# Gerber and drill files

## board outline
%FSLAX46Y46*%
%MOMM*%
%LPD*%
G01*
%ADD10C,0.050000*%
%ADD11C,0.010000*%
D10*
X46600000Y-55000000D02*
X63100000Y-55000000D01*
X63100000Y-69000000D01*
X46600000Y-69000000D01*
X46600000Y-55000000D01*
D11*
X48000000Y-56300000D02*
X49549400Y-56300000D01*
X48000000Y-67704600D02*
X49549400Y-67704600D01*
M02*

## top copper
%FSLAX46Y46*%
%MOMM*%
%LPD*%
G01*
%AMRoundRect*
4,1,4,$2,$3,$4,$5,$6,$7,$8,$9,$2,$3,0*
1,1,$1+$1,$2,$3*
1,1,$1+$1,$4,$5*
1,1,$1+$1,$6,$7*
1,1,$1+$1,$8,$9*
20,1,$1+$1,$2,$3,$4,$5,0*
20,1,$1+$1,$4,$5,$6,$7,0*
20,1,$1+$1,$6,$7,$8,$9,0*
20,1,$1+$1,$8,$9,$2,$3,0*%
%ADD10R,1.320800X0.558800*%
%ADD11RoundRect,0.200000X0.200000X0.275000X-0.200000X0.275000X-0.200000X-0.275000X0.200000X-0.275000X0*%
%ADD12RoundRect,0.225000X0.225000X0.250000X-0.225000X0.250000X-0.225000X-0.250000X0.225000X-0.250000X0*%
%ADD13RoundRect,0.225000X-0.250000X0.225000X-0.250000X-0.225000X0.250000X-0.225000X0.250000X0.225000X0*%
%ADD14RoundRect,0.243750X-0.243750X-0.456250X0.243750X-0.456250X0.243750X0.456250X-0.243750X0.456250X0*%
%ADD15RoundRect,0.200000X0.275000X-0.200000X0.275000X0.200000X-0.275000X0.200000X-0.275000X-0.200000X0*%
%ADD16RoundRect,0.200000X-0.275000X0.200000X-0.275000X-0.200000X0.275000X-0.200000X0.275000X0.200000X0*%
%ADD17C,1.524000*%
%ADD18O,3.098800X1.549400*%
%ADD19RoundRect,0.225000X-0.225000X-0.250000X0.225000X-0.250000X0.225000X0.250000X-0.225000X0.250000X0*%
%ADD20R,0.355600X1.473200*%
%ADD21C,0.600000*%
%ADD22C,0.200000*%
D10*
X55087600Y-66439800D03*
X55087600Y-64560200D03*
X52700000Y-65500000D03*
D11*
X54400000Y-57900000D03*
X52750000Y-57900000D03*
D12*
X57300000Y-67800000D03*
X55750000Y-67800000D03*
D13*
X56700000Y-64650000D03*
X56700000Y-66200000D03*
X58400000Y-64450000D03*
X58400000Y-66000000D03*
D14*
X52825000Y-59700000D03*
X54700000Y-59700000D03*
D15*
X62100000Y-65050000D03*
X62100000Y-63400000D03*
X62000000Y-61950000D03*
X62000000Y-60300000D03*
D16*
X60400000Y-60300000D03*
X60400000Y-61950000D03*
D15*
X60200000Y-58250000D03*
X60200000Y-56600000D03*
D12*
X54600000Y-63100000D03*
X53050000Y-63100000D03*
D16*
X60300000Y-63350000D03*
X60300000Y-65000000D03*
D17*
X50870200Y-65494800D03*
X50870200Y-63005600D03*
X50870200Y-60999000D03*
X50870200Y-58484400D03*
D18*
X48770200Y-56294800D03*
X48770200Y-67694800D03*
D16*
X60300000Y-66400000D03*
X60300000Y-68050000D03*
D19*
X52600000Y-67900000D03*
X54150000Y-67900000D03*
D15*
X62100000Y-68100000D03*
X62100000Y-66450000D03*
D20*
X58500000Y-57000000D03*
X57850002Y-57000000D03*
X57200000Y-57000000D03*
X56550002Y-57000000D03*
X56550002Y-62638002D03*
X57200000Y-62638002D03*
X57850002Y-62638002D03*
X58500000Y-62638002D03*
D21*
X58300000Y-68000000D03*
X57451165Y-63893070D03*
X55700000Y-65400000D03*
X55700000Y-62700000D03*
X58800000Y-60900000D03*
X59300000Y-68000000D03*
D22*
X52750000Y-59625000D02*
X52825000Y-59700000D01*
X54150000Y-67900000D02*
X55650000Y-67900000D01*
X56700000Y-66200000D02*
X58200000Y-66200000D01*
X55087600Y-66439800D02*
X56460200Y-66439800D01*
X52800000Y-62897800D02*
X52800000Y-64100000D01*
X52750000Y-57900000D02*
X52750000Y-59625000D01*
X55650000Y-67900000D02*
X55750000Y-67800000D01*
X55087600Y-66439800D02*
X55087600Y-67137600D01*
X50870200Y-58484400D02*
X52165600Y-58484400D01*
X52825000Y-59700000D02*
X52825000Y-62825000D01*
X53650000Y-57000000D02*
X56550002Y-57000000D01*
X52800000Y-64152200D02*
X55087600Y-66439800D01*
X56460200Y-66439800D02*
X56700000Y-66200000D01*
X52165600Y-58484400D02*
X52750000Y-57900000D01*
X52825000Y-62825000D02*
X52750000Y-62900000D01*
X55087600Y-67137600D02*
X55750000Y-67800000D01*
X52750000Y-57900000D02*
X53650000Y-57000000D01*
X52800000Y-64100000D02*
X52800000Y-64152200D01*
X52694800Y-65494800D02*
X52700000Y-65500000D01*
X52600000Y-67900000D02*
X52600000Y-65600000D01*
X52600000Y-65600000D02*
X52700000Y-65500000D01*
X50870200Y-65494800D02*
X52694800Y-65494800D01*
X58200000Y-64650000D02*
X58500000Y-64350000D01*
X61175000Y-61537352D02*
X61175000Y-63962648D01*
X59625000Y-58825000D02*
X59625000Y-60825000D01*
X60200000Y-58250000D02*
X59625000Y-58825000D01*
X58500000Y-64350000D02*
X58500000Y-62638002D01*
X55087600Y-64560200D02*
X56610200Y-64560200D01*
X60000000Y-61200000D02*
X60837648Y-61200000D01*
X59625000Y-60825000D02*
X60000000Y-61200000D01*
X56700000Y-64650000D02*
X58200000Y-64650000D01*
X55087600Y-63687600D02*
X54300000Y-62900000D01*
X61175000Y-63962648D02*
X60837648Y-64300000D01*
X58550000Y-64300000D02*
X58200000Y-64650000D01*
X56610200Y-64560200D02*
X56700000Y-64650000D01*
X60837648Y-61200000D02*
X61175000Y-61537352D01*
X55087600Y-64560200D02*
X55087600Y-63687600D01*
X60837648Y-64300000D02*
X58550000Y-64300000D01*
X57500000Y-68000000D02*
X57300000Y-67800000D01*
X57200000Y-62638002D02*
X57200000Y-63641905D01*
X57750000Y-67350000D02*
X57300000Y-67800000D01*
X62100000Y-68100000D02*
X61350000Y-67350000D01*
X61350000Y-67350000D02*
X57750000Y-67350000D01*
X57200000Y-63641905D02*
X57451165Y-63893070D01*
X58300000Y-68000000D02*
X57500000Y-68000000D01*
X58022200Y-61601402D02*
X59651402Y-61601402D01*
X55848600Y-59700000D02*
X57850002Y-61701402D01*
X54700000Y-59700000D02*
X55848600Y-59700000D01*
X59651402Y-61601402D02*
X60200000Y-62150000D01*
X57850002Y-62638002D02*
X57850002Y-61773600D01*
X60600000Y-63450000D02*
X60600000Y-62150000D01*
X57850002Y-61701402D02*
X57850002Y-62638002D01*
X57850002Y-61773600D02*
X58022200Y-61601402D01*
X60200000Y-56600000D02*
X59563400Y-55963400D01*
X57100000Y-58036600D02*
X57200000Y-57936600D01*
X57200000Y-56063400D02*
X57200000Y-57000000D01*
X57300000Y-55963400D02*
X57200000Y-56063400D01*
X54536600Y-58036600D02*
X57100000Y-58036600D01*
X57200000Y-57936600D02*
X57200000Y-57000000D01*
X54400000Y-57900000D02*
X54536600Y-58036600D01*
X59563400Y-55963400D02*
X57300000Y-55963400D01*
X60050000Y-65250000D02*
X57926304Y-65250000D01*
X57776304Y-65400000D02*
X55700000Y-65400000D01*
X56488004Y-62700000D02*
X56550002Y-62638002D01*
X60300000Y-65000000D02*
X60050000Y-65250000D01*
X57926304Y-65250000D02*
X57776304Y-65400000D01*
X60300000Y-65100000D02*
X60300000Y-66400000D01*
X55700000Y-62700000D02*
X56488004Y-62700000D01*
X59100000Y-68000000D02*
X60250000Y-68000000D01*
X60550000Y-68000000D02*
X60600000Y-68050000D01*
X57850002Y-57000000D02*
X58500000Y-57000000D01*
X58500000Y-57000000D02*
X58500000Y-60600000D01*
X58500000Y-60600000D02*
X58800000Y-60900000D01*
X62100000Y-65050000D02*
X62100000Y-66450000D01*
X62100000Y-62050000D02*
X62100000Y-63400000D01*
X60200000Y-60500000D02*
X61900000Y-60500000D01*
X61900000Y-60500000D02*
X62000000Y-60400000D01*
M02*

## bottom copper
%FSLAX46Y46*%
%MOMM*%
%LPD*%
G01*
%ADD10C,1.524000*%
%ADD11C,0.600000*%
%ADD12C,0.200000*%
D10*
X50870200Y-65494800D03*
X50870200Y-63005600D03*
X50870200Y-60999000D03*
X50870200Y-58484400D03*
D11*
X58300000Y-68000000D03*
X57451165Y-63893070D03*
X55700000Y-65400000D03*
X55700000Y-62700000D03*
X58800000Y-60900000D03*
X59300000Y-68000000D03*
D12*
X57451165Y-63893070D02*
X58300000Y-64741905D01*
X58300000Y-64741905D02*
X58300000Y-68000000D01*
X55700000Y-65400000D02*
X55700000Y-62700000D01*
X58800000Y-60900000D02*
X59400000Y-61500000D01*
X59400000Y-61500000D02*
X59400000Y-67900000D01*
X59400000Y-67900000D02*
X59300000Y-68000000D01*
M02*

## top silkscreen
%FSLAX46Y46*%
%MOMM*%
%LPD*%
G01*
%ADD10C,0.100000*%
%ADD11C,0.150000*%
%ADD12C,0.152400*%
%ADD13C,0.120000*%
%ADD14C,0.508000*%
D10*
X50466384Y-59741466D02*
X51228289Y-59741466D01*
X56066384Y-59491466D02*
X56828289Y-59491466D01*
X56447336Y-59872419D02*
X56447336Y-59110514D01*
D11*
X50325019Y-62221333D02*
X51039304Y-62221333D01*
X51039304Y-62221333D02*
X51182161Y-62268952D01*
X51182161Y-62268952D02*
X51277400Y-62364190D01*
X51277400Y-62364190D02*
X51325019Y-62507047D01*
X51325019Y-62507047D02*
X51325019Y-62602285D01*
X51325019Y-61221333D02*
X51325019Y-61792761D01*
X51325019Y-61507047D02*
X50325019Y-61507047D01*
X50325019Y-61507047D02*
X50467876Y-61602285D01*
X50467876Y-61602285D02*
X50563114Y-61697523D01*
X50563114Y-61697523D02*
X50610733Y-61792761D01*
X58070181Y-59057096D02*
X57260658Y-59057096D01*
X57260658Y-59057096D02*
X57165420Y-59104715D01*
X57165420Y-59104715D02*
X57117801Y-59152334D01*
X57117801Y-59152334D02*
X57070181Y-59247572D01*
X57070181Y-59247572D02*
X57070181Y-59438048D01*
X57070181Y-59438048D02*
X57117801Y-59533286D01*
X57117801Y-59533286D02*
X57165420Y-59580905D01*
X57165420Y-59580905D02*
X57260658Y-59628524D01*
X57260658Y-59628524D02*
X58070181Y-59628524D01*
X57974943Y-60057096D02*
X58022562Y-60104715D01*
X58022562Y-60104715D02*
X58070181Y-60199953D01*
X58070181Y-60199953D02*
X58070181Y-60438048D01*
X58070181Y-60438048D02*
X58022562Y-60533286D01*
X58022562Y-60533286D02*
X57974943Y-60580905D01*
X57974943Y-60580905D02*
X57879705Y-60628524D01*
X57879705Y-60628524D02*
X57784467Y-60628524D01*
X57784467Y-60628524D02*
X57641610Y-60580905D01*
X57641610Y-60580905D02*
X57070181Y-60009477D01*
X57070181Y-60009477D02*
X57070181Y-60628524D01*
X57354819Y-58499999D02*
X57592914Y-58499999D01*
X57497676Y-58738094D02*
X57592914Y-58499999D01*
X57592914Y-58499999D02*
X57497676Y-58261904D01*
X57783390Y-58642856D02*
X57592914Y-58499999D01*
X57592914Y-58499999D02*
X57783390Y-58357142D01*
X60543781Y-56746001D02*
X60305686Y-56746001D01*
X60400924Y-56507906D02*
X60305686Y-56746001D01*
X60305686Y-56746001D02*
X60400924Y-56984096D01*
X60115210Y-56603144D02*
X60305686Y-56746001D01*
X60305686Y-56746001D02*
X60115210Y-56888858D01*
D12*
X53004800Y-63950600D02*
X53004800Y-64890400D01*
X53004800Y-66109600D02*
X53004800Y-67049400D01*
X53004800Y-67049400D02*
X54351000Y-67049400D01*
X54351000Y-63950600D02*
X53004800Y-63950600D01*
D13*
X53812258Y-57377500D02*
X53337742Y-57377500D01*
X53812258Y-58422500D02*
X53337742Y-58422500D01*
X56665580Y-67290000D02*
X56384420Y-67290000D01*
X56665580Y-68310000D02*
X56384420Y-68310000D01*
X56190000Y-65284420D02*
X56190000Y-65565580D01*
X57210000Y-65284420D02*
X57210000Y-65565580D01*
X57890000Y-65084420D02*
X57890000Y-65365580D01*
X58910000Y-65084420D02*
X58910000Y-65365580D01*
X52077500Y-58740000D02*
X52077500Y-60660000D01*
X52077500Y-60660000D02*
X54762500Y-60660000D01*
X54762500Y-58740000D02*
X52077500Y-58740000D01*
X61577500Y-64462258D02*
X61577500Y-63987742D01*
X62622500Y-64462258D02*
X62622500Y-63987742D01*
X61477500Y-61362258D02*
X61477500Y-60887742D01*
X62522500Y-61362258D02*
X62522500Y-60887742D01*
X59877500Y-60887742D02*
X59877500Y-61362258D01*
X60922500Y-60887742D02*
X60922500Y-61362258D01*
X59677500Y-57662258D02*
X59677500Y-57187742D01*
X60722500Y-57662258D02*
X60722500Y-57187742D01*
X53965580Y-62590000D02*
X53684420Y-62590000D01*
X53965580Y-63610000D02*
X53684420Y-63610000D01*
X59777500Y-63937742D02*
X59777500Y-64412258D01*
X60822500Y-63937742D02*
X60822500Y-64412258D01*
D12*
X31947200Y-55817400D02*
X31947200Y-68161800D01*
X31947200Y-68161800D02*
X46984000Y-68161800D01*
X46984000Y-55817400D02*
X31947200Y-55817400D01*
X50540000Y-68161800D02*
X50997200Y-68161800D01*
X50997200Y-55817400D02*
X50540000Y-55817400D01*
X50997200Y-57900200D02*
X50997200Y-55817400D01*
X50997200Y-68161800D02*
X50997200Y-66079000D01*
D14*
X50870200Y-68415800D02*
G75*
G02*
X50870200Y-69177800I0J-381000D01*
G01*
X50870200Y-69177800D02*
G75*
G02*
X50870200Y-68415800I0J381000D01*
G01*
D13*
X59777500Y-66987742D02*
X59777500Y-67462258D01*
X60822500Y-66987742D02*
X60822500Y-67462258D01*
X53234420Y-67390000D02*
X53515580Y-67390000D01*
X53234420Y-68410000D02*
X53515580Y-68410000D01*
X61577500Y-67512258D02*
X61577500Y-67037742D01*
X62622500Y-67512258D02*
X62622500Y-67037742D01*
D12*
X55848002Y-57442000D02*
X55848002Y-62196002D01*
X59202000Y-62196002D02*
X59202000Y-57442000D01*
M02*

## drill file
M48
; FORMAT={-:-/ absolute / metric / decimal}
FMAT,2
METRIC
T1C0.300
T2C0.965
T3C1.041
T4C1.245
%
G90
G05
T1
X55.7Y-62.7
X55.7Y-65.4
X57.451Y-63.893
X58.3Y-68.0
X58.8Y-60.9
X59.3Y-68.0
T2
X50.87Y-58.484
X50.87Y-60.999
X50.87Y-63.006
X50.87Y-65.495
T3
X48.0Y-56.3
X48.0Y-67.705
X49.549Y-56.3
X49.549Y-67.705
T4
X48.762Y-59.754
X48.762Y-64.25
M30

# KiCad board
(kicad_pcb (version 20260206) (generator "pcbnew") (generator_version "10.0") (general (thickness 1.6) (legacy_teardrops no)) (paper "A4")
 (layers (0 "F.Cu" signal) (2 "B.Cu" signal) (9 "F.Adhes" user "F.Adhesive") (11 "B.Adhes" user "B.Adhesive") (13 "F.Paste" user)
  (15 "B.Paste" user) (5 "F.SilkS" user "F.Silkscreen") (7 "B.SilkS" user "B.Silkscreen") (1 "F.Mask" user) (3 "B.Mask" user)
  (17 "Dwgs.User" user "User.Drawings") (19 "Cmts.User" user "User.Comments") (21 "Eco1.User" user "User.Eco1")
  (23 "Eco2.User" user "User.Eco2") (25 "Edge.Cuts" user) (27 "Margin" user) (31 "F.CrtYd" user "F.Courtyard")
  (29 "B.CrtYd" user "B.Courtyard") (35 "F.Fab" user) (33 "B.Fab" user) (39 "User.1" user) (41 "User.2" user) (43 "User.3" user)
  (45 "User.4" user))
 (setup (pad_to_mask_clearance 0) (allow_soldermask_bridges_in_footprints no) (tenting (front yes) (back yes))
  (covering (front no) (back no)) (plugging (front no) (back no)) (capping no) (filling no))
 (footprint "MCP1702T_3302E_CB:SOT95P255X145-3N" (layer "F.Cu") (at 53.8938 65.5 90)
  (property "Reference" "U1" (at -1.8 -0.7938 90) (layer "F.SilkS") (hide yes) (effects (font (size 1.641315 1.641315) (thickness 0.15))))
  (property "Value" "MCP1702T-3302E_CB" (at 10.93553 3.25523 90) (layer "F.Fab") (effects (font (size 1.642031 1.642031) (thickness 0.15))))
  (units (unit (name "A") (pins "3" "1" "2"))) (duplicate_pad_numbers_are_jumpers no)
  (fp_line (start 1.5494 -0.889) (end 0.6096 -0.889) (stroke (width 0.1524) (type solid)) (layer "F.SilkS"))
  (fp_line (start -0.6096 -0.889) (end -1.5494 -0.889) (stroke (width 0.1524) (type solid)) (layer "F.SilkS"))
  (fp_line (start -1.5494 -0.889) (end -1.5494 0.4572) (stroke (width 0.1524) (type solid)) (layer "F.SilkS"))
  (fp_line (start 1.5494 0.4572) (end 1.5494 -0.889) (stroke (width 0.1524) (type solid)) (layer "F.SilkS"))
  (pad "1" smd rect (at -0.9398 1.1938 90) (size 0.5588 1.3208) (layers "F.Cu" "F.Mask" "F.Paste") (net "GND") (solder_mask_margin 0.102))
  (pad "2" smd rect (at 0.9398 1.1938 90) (size 0.5588 1.3208) (layers "F.Cu" "F.Mask" "F.Paste") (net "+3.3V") (solder_mask_margin 0.102))
  (pad "3" smd rect (at 0 -1.1938 90) (size 0.5588 1.3208) (layers "F.Cu" "F.Mask" "F.Paste") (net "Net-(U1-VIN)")
   (solder_mask_margin 0.102)))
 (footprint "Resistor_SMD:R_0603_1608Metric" (layer "F.Cu") (at 53.575 57.9 180)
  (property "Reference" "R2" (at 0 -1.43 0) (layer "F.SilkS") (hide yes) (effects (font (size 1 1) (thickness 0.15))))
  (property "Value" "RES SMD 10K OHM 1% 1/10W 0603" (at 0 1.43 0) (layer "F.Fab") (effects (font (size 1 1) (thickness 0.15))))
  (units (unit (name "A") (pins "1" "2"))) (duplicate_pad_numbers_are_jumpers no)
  (fp_line (start -0.237258 0.5225) (end 0.237258 0.5225) (stroke (width 0.12) (type solid)) (layer "F.SilkS"))
  (fp_line (start -0.237258 -0.5225) (end 0.237258 -0.5225) (stroke (width 0.12) (type solid)) (layer "F.SilkS"))
  (pad "1" smd roundrect (at -0.825 0 180) (size 0.8 0.95) (layers "F.Cu" "F.Mask" "F.Paste") (roundrect_rratio 0.25) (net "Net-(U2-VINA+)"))
  (pad "2" smd roundrect (at 0.825 0 180) (size 0.8 0.95) (layers "F.Cu" "F.Mask" "F.Paste") (roundrect_rratio 0.25) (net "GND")))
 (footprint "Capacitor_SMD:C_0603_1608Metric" (layer "F.Cu") (at 56.525 67.8 180)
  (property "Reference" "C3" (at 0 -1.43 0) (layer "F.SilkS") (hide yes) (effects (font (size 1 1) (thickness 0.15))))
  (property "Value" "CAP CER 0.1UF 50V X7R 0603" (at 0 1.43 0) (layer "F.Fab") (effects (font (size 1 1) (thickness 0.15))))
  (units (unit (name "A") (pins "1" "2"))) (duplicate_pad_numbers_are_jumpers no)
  (fp_line (start -0.14058 0.51) (end 0.14058 0.51) (stroke (width 0.12) (type solid)) (layer "F.SilkS"))
  (fp_line (start -0.14058 -0.51) (end 0.14058 -0.51) (stroke (width 0.12) (type solid)) (layer "F.SilkS"))
  (pad "1" smd roundrect (at -0.775 0 180) (size 0.9 0.95) (layers "F.Cu" "F.Mask" "F.Paste") (roundrect_rratio 0.25) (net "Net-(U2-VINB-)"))
  (pad "2" smd roundrect (at 0.775 0 180) (size 0.9 0.95) (layers "F.Cu" "F.Mask" "F.Paste") (roundrect_rratio 0.25) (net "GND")))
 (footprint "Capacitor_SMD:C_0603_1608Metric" (layer "F.Cu") (at 56.7 65.425 -90)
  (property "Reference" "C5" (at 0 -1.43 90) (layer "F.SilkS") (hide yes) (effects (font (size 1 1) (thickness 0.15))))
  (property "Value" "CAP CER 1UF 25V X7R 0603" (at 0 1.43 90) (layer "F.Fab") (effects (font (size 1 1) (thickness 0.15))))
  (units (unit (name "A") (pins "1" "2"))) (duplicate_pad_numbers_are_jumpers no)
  (fp_line (start -0.14058 0.51) (end 0.14058 0.51) (stroke (width 0.12) (type solid)) (layer "F.SilkS"))
  (fp_line (start -0.14058 -0.51) (end 0.14058 -0.51) (stroke (width 0.12) (type solid)) (layer "F.SilkS"))
  (pad "1" smd roundrect (at -0.775 0 270) (size 0.9 0.95) (layers "F.Cu" "F.Mask" "F.Paste") (roundrect_rratio 0.25) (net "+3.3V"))
  (pad "2" smd roundrect (at 0.775 0 270) (size 0.9 0.95) (layers "F.Cu" "F.Mask" "F.Paste") (roundrect_rratio 0.25) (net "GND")))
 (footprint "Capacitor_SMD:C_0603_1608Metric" (layer "F.Cu") (at 58.4 65.225 -90)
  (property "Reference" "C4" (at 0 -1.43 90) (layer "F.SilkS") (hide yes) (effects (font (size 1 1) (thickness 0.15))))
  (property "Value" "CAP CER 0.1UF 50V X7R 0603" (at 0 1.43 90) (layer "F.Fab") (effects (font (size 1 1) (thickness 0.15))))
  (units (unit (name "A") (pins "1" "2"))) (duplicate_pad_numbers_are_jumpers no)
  (fp_line (start -0.14058 0.51) (end 0.14058 0.51) (stroke (width 0.12) (type solid)) (layer "F.SilkS"))
  (fp_line (start -0.14058 -0.51) (end 0.14058 -0.51) (stroke (width 0.12) (type solid)) (layer "F.SilkS"))
  (pad "1" smd roundrect (at -0.775 0 270) (size 0.9 0.95) (layers "F.Cu" "F.Mask" "F.Paste") (roundrect_rratio 0.25) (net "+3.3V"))
  (pad "2" smd roundrect (at 0.775 0 270) (size 0.9 0.95) (layers "F.Cu" "F.Mask" "F.Paste") (roundrect_rratio 0.25) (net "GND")))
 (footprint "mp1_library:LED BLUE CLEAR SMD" (layer "F.Cu") (at 53.7625 59.7)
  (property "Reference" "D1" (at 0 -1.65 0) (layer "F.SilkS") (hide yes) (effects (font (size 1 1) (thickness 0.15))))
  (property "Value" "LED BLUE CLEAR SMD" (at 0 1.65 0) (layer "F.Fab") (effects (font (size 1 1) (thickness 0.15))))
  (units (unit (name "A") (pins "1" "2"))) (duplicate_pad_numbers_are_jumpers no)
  (fp_line (start -1.685 -0.96) (end -1.685 0.96) (stroke (width 0.12) (type solid)) (layer "F.SilkS"))
  (fp_line (start -1.685 0.96) (end 1 0.96) (stroke (width 0.12) (type solid)) (layer "F.SilkS"))
  (fp_line (start 1 -0.96) (end -1.685 -0.96) (stroke (width 0.12) (type solid)) (layer "F.SilkS"))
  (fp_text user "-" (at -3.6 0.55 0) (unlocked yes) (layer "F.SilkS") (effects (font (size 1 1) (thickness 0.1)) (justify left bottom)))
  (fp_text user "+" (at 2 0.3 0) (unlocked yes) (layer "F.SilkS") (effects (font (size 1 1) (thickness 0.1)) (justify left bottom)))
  (pad "1" smd roundrect (at -0.9375 0) (size 0.975 1.4) (layers "F.Cu" "F.Mask" "F.Paste") (roundrect_rratio 0.25) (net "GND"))
  (pad "2" smd roundrect (at 0.9375 0) (size 0.975 1.4) (layers "F.Cu" "F.Mask" "F.Paste") (roundrect_rratio 0.25) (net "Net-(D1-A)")))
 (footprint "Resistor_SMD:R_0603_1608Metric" (layer "F.Cu") (at 62.1 64.225 90)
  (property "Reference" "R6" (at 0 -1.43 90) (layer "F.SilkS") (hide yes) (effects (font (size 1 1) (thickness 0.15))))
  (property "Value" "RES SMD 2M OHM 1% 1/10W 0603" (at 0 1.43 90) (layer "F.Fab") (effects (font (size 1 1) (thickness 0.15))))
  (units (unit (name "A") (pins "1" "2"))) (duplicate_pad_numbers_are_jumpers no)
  (fp_line (start -0.237258 -0.5225) (end 0.237258 -0.5225) (stroke (width 0.12) (type solid)) (layer "F.SilkS"))
  (fp_line (start -0.237258 0.5225) (end 0.237258 0.5225) (stroke (width 0.12) (type solid)) (layer "F.SilkS"))
  (pad "1" smd roundrect (at -0.825 0 90) (size 0.8 0.95) (layers "F.Cu" "F.Mask" "F.Paste") (roundrect_rratio 0.25) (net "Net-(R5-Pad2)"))
  (pad "2" smd roundrect (at 0.825 0 90) (size 0.8 0.95) (layers "F.Cu" "F.Mask" "F.Paste") (roundrect_rratio 0.25) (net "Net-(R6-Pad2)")))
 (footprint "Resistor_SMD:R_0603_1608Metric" (layer "F.Cu") (at 62 61.125 90)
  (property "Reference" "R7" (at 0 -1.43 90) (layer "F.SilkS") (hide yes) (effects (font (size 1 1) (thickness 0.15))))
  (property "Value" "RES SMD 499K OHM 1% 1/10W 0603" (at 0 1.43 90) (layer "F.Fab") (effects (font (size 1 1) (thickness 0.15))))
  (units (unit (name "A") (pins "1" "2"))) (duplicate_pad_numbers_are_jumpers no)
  (fp_line (start -0.237258 -0.5225) (end 0.237258 -0.5225) (stroke (width 0.12) (type solid)) (layer "F.SilkS"))
  (fp_line (start -0.237258 0.5225) (end 0.237258 0.5225) (stroke (width 0.12) (type solid)) (layer "F.SilkS"))
  (pad "1" smd roundrect (at -0.825 0 90) (size 0.8 0.95) (layers "F.Cu" "F.Mask" "F.Paste") (roundrect_rratio 0.25) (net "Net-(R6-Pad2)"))
  (pad "2" smd roundrect (at 0.825 0 90) (size 0.8 0.95) (layers "F.Cu" "F.Mask" "F.Paste") (roundrect_rratio 0.25) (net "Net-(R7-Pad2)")))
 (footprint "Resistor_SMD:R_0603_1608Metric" (layer "F.Cu") (at 60.4 61.125 -90)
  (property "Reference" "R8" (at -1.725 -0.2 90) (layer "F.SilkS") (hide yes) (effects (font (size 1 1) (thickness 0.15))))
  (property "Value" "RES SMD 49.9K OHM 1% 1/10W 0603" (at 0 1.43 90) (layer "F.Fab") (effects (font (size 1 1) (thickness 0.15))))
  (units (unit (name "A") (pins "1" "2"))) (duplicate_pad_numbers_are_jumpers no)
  (fp_line (start -0.237258 0.5225) (end 0.237258 0.5225) (stroke (width 0.12) (type solid)) (layer "F.SilkS"))
  (fp_line (start -0.237258 -0.5225) (end 0.237258 -0.5225) (stroke (width 0.12) (type solid)) (layer "F.SilkS"))
  (pad "1" smd roundrect (at -0.825 0 270) (size 0.8 0.95) (layers "F.Cu" "F.Mask" "F.Paste") (roundrect_rratio 0.25) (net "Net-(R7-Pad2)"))
  (pad "2" smd roundrect (at 0.825 0 270) (size 0.8 0.95) (layers "F.Cu" "F.Mask" "F.Paste") (roundrect_rratio 0.25) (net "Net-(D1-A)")))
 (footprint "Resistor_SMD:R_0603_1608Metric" (layer "F.Cu") (at 60.2 57.425 90)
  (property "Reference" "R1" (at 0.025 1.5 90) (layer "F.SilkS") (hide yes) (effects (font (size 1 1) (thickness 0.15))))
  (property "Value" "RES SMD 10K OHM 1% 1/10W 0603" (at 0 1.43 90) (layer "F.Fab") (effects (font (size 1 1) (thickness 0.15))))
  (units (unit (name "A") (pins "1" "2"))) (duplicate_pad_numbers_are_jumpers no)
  (fp_line (start -0.237258 -0.5225) (end 0.237258 -0.5225) (stroke (width 0.12) (type solid)) (layer "F.SilkS"))
  (fp_line (start -0.237258 0.5225) (end 0.237258 0.5225) (stroke (width 0.12) (type solid)) (layer "F.SilkS"))
  (pad "1" smd roundrect (at -0.825 0 90) (size 0.8 0.95) (layers "F.Cu" "F.Mask" "F.Paste") (roundrect_rratio 0.25) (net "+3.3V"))
  (pad "2" smd roundrect (at 0.825 0 90) (size 0.8 0.95) (layers "F.Cu" "F.Mask" "F.Paste") (roundrect_rratio 0.25) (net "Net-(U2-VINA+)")))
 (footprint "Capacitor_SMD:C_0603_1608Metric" (layer "F.Cu") (at 53.825 63.1 180)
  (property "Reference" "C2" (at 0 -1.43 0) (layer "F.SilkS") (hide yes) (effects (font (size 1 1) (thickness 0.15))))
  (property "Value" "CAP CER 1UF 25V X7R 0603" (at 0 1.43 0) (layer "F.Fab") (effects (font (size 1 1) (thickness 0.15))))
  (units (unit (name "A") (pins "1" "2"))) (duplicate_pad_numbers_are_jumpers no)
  (fp_line (start -0.14058 0.51) (end 0.14058 0.51) (stroke (width 0.12) (type solid)) (layer "F.SilkS"))
  (fp_line (start -0.14058 -0.51) (end 0.14058 -0.51) (stroke (width 0.12) (type solid)) (layer "F.SilkS"))
  (pad "1" smd roundrect (at -0.775 0 180) (size 0.9 0.95) (layers "F.Cu" "F.Mask" "F.Paste") (roundrect_rratio 0.25) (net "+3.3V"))
  (pad "2" smd roundrect (at 0.775 0 180) (size 0.9 0.95) (layers "F.Cu" "F.Mask" "F.Paste") (roundrect_rratio 0.25) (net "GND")))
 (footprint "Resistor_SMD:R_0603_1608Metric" (layer "F.Cu") (at 60.3 64.175 -90)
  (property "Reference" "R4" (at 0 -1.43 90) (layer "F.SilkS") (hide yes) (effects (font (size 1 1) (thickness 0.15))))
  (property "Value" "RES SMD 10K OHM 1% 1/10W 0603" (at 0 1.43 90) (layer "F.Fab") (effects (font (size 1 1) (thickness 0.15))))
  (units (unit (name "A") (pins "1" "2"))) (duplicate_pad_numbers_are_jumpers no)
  (fp_line (start -0.237258 0.5225) (end 0.237258 0.5225) (stroke (width 0.12) (type solid)) (layer "F.SilkS"))
  (fp_line (start -0.237258 -0.5225) (end 0.237258 -0.5225) (stroke (width 0.12) (type solid)) (layer "F.SilkS"))
  (pad "1" smd roundrect (at -0.825 0 270) (size 0.8 0.95) (layers "F.Cu" "F.Mask" "F.Paste") (roundrect_rratio 0.25) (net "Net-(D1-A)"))
  (pad "2" smd roundrect (at 0.825 0 270) (size 0.8 0.95) (layers "F.Cu" "F.Mask" "F.Paste") (roundrect_rratio 0.25) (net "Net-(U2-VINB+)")))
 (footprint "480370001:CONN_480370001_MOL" (layer "F.Cu") (at 50.8702 65.4948 -90)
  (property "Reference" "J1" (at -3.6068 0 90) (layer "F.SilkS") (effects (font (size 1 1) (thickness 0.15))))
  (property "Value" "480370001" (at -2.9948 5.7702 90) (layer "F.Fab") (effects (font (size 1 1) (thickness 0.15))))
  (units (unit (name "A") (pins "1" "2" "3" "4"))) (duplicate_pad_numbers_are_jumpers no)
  (fp_line (start -9.6774 18.923) (end 2.667 18.923) (stroke (width 0.1524) (type solid)) (layer "F.SilkS"))
  (fp_line (start 2.667 18.923) (end 2.667 3.8862) (stroke (width 0.1524) (type solid)) (layer "F.SilkS"))
  (fp_line (start -9.6774 3.8862) (end -9.6774 18.923) (stroke (width 0.1524) (type solid)) (layer "F.SilkS"))
  (fp_line (start 2.667 0.3302) (end 2.667 -0.127) (stroke (width 0.1524) (type solid)) (layer "F.SilkS"))
  (fp_line (start -9.6774 -0.127) (end -9.6774 0.3302) (stroke (width 0.1524) (type solid)) (layer "F.SilkS"))
  (fp_line (start -7.5946 -0.127) (end -9.6774 -0.127) (stroke (width 0.1524) (type solid)) (layer "F.SilkS"))
  (fp_line (start 2.667 -0.127) (end 0.5842 -0.127) (stroke (width 0.1524) (type solid)) (layer "F.SilkS"))
  (fp_arc (start 2.921 0) (mid 3.302 -0.381) (end 3.683 0) (stroke (width 0.508) (type solid)) (layer "F.SilkS"))
  (fp_arc (start 3.683 0) (mid 3.302 0.381) (end 2.921 0) (stroke (width 0.508) (type solid)) (layer "F.SilkS"))
  (fp_line (start -9.1948 2.8702) (end -9.1948 1.3208) (stroke (width 0.01) (type solid)) (layer "Edge.Cuts"))
  (fp_line (start 2.2098 2.8702) (end 2.2098 1.3208) (stroke (width 0.01) (type solid)) (layer "Edge.Cuts"))
  (pad "" np_thru_hole circle (at -9.1948 1.3208 270) (size 1.0414 1.0414) (drill 1.0414) (layers "*.Cu" "*.Mask"))
  (pad "" np_thru_hole circle (at -9.1948 2.8702 270) (size 1.0414 1.0414) (drill 1.0414) (layers "*.Cu" "*.Mask"))
  (pad "" np_thru_hole circle (at -5.7404 2.1082 270) (size 1.2446 1.2446) (drill 1.2446) (layers "*.Cu" "*.Mask"))
  (pad "" np_thru_hole circle (at -1.2446 2.1082 270) (size 1.2446 1.2446) (drill 1.2446) (layers "*.Cu" "*.Mask"))
  (pad "" np_thru_hole circle (at 2.2098 1.3208 270) (size 1.0414 1.0414) (drill 1.0414) (layers "*.Cu" "*.Mask"))
  (pad "" np_thru_hole circle (at 2.2098 2.8702 270) (size 1.0414 1.0414) (drill 1.0414) (layers "*.Cu" "*.Mask"))
  (pad "1" thru_hole circle (at 0 0 270) (size 1.524 1.524) (drill 0.9652) (layers "*.Cu" "*.Mask") (remove_unused_layers no)
   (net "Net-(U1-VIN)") (solder_mask_margin 0.102))
  (pad "2" thru_hole circle (at -2.4892 0 270) (size 1.524 1.524) (drill 0.9652) (layers "*.Cu" "*.Mask") (remove_unused_layers no)
   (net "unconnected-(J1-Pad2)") (solder_mask_margin 0.102))
  (pad "3" thru_hole circle (at -4.4958 0 270) (size 1.524 1.524) (drill 0.9652) (layers "*.Cu" "*.Mask") (remove_unused_layers no)
   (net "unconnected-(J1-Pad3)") (solder_mask_margin 0.102))
  (pad "4" thru_hole circle (at -7.0104 0 270) (size 1.524 1.524) (drill 0.9652) (layers "*.Cu" "*.Mask") (remove_unused_layers no)
   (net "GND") (solder_mask_margin 0.102))
  (pad "7" smd oval (at -9.2 2.1 270) (size 1.5494 3.0988) (layers "F.Cu" "F.Mask" "F.Paste") (solder_mask_margin 0.102))
  (pad "8" smd oval (at 2.2 2.1 270) (size 1.5494 3.0988) (layers "F.Cu" "F.Mask" "F.Paste") (solder_mask_margin 0.102)))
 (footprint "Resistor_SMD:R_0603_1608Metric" (layer "F.Cu") (at 60.3 67.225 -90)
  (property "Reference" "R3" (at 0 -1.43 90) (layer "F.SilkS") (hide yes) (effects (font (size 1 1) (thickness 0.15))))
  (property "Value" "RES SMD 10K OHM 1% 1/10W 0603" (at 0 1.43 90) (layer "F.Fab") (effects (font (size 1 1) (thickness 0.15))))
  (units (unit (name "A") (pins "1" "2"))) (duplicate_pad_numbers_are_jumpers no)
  (fp_line (start -0.237258 0.5225) (end 0.237258 0.5225) (stroke (width 0.12) (type solid)) (layer "F.SilkS"))
  (fp_line (start -0.237258 -0.5225) (end 0.237258 -0.5225) (stroke (width 0.12) (type solid)) (layer "F.SilkS"))
  (pad "1" smd roundrect (at -0.825 0 270) (size 0.8 0.95) (layers "F.Cu" "F.Mask" "F.Paste") (roundrect_rratio 0.25) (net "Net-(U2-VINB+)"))
  (pad "2" smd roundrect (at 0.825 0 270) (size 0.8 0.95) (layers "F.Cu" "F.Mask" "F.Paste") (roundrect_rratio 0.25) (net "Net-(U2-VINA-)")))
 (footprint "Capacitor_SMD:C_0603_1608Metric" (layer "F.Cu") (at 53.375 67.9)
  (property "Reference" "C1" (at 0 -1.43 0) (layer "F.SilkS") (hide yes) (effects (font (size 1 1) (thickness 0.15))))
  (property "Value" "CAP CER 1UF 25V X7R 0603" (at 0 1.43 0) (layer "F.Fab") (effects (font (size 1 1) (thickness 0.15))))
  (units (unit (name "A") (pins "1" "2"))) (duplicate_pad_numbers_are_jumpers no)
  (fp_line (start -0.14058 -0.51) (end 0.14058 -0.51) (stroke (width 0.12) (type solid)) (layer "F.SilkS"))
  (fp_line (start -0.14058 0.51) (end 0.14058 0.51) (stroke (width 0.12) (type solid)) (layer "F.SilkS"))
  (pad "1" smd roundrect (at -0.775 0) (size 0.9 0.95) (layers "F.Cu" "F.Mask" "F.Paste") (roundrect_rratio 0.25) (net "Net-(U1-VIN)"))
  (pad "2" smd roundrect (at 0.775 0) (size 0.9 0.95) (layers "F.Cu" "F.Mask" "F.Paste") (roundrect_rratio 0.25) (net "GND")))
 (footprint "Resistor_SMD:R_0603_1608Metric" (layer "F.Cu") (at 62.1 67.275 90)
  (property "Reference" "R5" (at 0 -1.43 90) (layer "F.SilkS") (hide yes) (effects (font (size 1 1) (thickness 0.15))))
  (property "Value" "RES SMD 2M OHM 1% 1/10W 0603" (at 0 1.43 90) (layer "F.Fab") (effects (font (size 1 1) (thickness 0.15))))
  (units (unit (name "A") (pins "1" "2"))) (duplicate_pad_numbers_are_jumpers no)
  (fp_line (start -0.237258 -0.5225) (end 0.237258 -0.5225) (stroke (width 0.12) (type solid)) (layer "F.SilkS"))
  (fp_line (start -0.237258 0.5225) (end 0.237258 0.5225) (stroke (width 0.12) (type solid)) (layer "F.SilkS"))
  (pad "1" smd roundrect (at -0.825 0 90) (size 0.8 0.95) (layers "F.Cu" "F.Mask" "F.Paste") (roundrect_rratio 0.25) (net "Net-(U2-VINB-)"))
  (pad "2" smd roundrect (at 0.825 0 90) (size 0.8 0.95) (layers "F.Cu" "F.Mask" "F.Paste") (roundrect_rratio 0.25) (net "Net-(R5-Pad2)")))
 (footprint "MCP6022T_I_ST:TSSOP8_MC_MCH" (layer "F.Cu") (at 57.525001 59.819001 -90)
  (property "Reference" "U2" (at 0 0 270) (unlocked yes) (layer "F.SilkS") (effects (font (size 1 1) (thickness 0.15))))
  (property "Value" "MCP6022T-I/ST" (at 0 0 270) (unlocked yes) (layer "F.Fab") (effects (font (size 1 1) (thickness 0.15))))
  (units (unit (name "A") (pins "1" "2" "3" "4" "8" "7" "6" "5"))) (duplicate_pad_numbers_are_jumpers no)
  (fp_line (start -2.377001 1.676999) (end 2.377001 1.676999) (stroke (width 0.1524) (type solid)) (layer "F.SilkS"))
  (fp_line (start 2.377001 -1.676999) (end -2.377001 -1.676999) (stroke (width 0.1524) (type solid)) (layer "F.SilkS"))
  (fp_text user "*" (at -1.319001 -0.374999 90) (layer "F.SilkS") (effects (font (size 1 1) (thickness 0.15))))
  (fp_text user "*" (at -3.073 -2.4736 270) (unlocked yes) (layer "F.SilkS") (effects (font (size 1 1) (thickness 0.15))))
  (pad "1" smd rect (at -2.819001 -0.974999 270) (size 1.4732 0.3556) (layers "F.Cu" "F.Mask" "F.Paste") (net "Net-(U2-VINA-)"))
  (pad "2" smd rect (at -2.819001 -0.325001 270) (size 1.4732 0.3556) (layers "F.Cu" "F.Mask" "F.Paste") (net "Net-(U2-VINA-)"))
  (pad "3" smd rect (at -2.819001 0.325001 270) (size 1.4732 0.3556) (layers "F.Cu" "F.Mask" "F.Paste") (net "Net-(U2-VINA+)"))
  (pad "4" smd rect (at -2.819001 0.974999 270) (size 1.4732 0.3556) (layers "F.Cu" "F.Mask" "F.Paste") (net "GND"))
  (pad "5" smd rect (at 2.819001 0.974999 270) (size 1.4732 0.3556) (layers "F.Cu" "F.Mask" "F.Paste") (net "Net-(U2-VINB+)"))
  (pad "6" smd rect (at 2.819001 0.325001 270) (size 1.4732 0.3556) (layers "F.Cu" "F.Mask" "F.Paste") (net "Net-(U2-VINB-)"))
  (pad "7" smd rect (at 2.819001 -0.325001 270) (size 1.4732 0.3556) (layers "F.Cu" "F.Mask" "F.Paste") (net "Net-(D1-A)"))
  (pad "8" smd rect (at 2.819001 -0.974999 270) (size 1.4732 0.3556) (layers "F.Cu" "F.Mask" "F.Paste") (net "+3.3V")))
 (gr_rect (start 46.6 55) (end 63.1 69) (stroke (width 0.05) (type default)) (fill no) (layer "Edge.Cuts"))
 (segment (start 52.75 59.625) (end 52.825 59.7) (width 0.2) (layer "F.Cu") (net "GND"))
 (segment (start 54.15 67.9) (end 55.65 67.9) (width 0.2) (layer "F.Cu") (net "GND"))
 (segment (start 56.7 66.2) (end 58.2 66.2) (width 0.2) (layer "F.Cu") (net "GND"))
 (segment (start 55.0876 66.4398) (end 56.4602 66.4398) (width 0.2) (layer "F.Cu") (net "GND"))
 (segment (start 52.8 62.8978) (end 52.8 64.1) (width 0.2) (layer "F.Cu") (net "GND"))
 (segment (start 52.75 57.9) (end 52.75 59.625) (width 0.2) (layer "F.Cu") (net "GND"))
 (segment (start 55.65 67.9) (end 55.75 67.8) (width 0.2) (layer "F.Cu") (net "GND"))
 (segment (start 55.0876 66.4398) (end 55.0876 67.1376) (width 0.2) (layer "F.Cu") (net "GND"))
 (segment (start 50.8702 58.4844) (end 52.1656 58.4844) (width 0.2) (layer "F.Cu") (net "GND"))
 (segment (start 52.825 59.7) (end 52.825 62.825) (width 0.2) (layer "F.Cu") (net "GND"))
 (segment (start 53.65 57) (end 56.550002 57) (width 0.2) (layer "F.Cu") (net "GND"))
 (segment (start 52.8 64.1522) (end 55.0876 66.4398) (width 0.2) (layer "F.Cu") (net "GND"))
 (segment (start 56.4602 66.4398) (end 56.7 66.2) (width 0.2) (layer "F.Cu") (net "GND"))
 (segment (start 52.1656 58.4844) (end 52.75 57.9) (width 0.2) (layer "F.Cu") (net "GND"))
 (segment (start 52.825 62.825) (end 52.75 62.9) (width 0.2) (layer "F.Cu") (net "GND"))
 (segment (start 55.0876 67.1376) (end 55.75 67.8) (width 0.2) (layer "F.Cu") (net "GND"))
 (segment (start 52.75 57.9) (end 53.65 57) (width 0.2) (layer "F.Cu") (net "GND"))
 (segment (start 52.8 64.1) (end 52.8 64.1522) (width 0.2) (layer "F.Cu") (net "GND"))
 (segment (start 52.6948 65.4948) (end 52.7 65.5) (width 0.2) (layer "F.Cu") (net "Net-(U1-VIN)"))
 (segment (start 52.6 67.9) (end 52.6 65.6) (width 0.2) (layer "F.Cu") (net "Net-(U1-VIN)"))
 (segment (start 52.6 65.6) (end 52.7 65.5) (width 0.2) (layer "F.Cu") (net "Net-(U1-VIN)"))
 (segment (start 50.8702 65.4948) (end 52.6948 65.4948) (width 0.2) (layer "F.Cu") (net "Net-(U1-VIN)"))
 (segment (start 58.2 64.65) (end 58.5 64.35) (width 0.2) (layer "F.Cu") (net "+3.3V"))
 (segment (start 61.175 61.537352) (end 61.175 63.962648) (width 0.2) (layer "F.Cu") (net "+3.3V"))
 (segment (start 59.625 58.825) (end 59.625 60.825) (width 0.2) (layer "F.Cu") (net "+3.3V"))
 (segment (start 60.2 58.25) (end 59.625 58.825) (width 0.2) (layer "F.Cu") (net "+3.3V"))
 (segment (start 58.5 64.35) (end 58.5 62.638002) (width 0.2) (layer "F.Cu") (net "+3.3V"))
 (segment (start 55.0876 64.5602) (end 56.6102 64.5602) (width 0.2) (layer "F.Cu") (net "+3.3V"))
 (segment (start 60 61.2) (end 60.837648 61.2) (width 0.2) (layer "F.Cu") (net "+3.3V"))
 (segment (start 59.625 60.825) (end 60 61.2) (width 0.2) (layer "F.Cu") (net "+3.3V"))
 (segment (start 56.7 64.65) (end 58.2 64.65) (width 0.2) (layer "F.Cu") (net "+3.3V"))
 (segment (start 55.0876 63.6876) (end 54.3 62.9) (width 0.2) (layer "F.Cu") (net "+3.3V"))
 (segment (start 61.175 63.962648) (end 60.837648 64.3) (width 0.2) (layer "F.Cu") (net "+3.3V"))
 (segment (start 58.55 64.3) (end 58.2 64.65) (width 0.2) (layer "F.Cu") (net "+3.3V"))
 (segment (start 56.6102 64.5602) (end 56.7 64.65) (width 0.2) (layer "F.Cu") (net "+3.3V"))
 (segment (start 60.837648 61.2) (end 61.175 61.537352) (width 0.2) (layer "F.Cu") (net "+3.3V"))
 (segment (start 55.0876 64.5602) (end 55.0876 63.6876) (width 0.2) (layer "F.Cu") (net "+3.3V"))
 (segment (start 60.837648 64.3) (end 58.55 64.3) (width 0.2) (layer "F.Cu") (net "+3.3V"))
 (segment (start 57.5 68) (end 57.3 67.8) (width 0.2) (layer "F.Cu") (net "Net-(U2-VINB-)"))
 (segment (start 57.2 62.638002) (end 57.2 63.641905) (width 0.2) (layer "F.Cu") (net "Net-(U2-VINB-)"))
 (segment (start 57.75 67.35) (end 57.3 67.8) (width 0.2) (layer "F.Cu") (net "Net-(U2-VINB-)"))
 (segment (start 62.1 68.1) (end 61.35 67.35) (width 0.2) (layer "F.Cu") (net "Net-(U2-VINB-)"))
 (segment (start 61.35 67.35) (end 57.75 67.35) (width 0.2) (layer "F.Cu") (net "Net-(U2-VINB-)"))
 (segment (start 57.2 63.641905) (end 57.451165 63.89307) (width 0.2) (layer "F.Cu") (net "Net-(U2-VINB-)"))
 (segment (start 58.3 68) (end 57.5 68) (width 0.2) (layer "F.Cu") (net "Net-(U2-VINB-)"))
 (via (at 58.3 68) (size 0.6) (drill 0.3) (layers "F.Cu" "B.Cu") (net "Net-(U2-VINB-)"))
 (via (at 57.451165 63.89307) (size 0.6) (drill 0.3) (layers "F.Cu" "B.Cu") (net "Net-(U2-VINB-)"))
 (segment (start 57.451165 63.89307) (end 58.3 64.741905) (width 0.2) (layer "B.Cu") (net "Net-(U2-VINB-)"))
 (segment (start 58.3 64.741905) (end 58.3 68) (width 0.2) (layer "B.Cu") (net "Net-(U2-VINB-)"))
 (segment (start 58.0222 61.601402) (end 59.651402 61.601402) (width 0.2) (layer "F.Cu") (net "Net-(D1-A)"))
 (segment (start 55.8486 59.7) (end 57.850002 61.701402) (width 0.2) (layer "F.Cu") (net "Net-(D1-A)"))
 (segment (start 54.7 59.7) (end 55.8486 59.7) (width 0.2) (layer "F.Cu") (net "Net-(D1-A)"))
 (segment (start 59.651402 61.601402) (end 60.2 62.15) (width 0.2) (layer "F.Cu") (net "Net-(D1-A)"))
 (segment (start 57.850002 62.638002) (end 57.850002 61.7736) (width 0.2) (layer "F.Cu") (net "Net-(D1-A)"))
 (segment (start 60.6 63.45) (end 60.6 62.15) (width 0.2) (layer "F.Cu") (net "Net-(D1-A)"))
 (segment (start 57.850002 61.701402) (end 57.850002 62.638002) (width 0.2) (layer "F.Cu") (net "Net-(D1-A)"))
 (segment (start 57.850002 61.7736) (end 58.0222 61.601402) (width 0.2) (layer "F.Cu") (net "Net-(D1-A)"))
 (segment (start 60.2 56.6) (end 59.5634 55.9634) (width 0.2) (layer "F.Cu") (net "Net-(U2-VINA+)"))
 (segment (start 57.1 58.0366) (end 57.2 57.9366) (width 0.2) (layer "F.Cu") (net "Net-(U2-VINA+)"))
 (segment (start 57.2 56.0634) (end 57.2 57) (width 0.2) (layer "F.Cu") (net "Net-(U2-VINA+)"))
 (segment (start 57.3 55.9634) (end 57.2 56.0634) (width 0.2) (layer "F.Cu") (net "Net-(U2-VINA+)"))
 (segment (start 54.5366 58.0366) (end 57.1 58.0366) (width 0.2) (layer "F.Cu") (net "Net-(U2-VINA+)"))
 (segment (start 57.2 57.9366) (end 57.2 57) (width 0.2) (layer "F.Cu") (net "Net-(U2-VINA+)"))
 (segment (start 54.4 57.9) (end 54.5366 58.0366) (width 0.2) (layer "F.Cu") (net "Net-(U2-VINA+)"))
 (segment (start 59.5634 55.9634) (end 57.3 55.9634) (width 0.2) (layer "F.Cu") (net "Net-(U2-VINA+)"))
 (segment (start 60.05 65.25) (end 57.926304 65.25) (width 0.2) (layer "F.Cu") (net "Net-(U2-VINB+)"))
 (segment (start 57.776304 65.4) (end 55.7 65.4) (width 0.2) (layer "F.Cu") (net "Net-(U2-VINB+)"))
 (segment (start 56.488004 62.7) (end 56.550002 62.638002) (width 0.2) (layer "F.Cu") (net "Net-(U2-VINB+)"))
 (segment (start 60.3 65) (end 60.05 65.25) (width 0.2) (layer "F.Cu") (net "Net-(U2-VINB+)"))
 (segment (start 57.926304 65.25) (end 57.776304 65.4) (width 0.2) (layer "F.Cu") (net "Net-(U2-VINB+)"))
 (segment (start 60.3 65.1) (end 60.3 66.4) (width 0.2) (layer "F.Cu") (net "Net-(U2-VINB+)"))
 (segment (start 55.7 62.7) (end 56.488004 62.7) (width 0.2) (layer "F.Cu") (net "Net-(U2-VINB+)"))
 (via (at 55.7 65.4) (size 0.6) (drill 0.3) (layers "F.Cu" "B.Cu") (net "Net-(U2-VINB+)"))
 (via (at 55.7 62.7) (size 0.6) (drill 0.3) (layers "F.Cu" "B.Cu") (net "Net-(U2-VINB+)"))
 (segment (start 55.7 65.4) (end 55.7 62.7) (width 0.2) (layer "B.Cu") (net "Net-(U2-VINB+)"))
 (segment (start 59.1 68) (end 60.25 68) (width 0.2) (layer "F.Cu") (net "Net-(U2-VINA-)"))
 (segment (start 60.55 68) (end 60.6 68.05) (width 0.2) (layer "F.Cu") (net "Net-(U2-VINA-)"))
 (segment (start 57.850002 57) (end 58.5 57) (width 0.2) (layer "F.Cu") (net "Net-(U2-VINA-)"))
 (segment (start 58.5 57) (end 58.5 60.6) (width 0.2) (layer "F.Cu") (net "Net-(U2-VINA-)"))
 (segment (start 58.5 60.6) (end 58.8 60.9) (width 0.2) (layer "F.Cu") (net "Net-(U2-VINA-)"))
 (via (at 58.8 60.9) (size 0.6) (drill 0.3) (layers "F.Cu" "B.Cu") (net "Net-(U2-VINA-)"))
 (via (at 59.3 68) (size 0.6) (drill 0.3) (layers "F.Cu" "B.Cu") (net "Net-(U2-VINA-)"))
 (segment (start 58.8 60.9) (end 59.4 61.5) (width 0.2) (layer "B.Cu") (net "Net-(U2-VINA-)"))
 (segment (start 59.4 61.5) (end 59.4 67.9) (width 0.2) (layer "B.Cu") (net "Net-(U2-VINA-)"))
 (segment (start 59.4 67.9) (end 59.3 68) (width 0.2) (layer "B.Cu") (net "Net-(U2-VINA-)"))
 (segment (start 62.1 65.05) (end 62.1 66.45) (width 0.2) (layer "F.Cu") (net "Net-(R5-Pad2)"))
 (segment (start 62.1 62.05) (end 62.1 63.4) (width 0.2) (layer "F.Cu") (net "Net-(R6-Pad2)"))
 (segment (start 60.2 60.5) (end 61.9 60.5) (width 0.2) (layer "F.Cu") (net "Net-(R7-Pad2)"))
 (segment (start 61.9 60.5) (end 62 60.4) (width 0.2) (layer "F.Cu") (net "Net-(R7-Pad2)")))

